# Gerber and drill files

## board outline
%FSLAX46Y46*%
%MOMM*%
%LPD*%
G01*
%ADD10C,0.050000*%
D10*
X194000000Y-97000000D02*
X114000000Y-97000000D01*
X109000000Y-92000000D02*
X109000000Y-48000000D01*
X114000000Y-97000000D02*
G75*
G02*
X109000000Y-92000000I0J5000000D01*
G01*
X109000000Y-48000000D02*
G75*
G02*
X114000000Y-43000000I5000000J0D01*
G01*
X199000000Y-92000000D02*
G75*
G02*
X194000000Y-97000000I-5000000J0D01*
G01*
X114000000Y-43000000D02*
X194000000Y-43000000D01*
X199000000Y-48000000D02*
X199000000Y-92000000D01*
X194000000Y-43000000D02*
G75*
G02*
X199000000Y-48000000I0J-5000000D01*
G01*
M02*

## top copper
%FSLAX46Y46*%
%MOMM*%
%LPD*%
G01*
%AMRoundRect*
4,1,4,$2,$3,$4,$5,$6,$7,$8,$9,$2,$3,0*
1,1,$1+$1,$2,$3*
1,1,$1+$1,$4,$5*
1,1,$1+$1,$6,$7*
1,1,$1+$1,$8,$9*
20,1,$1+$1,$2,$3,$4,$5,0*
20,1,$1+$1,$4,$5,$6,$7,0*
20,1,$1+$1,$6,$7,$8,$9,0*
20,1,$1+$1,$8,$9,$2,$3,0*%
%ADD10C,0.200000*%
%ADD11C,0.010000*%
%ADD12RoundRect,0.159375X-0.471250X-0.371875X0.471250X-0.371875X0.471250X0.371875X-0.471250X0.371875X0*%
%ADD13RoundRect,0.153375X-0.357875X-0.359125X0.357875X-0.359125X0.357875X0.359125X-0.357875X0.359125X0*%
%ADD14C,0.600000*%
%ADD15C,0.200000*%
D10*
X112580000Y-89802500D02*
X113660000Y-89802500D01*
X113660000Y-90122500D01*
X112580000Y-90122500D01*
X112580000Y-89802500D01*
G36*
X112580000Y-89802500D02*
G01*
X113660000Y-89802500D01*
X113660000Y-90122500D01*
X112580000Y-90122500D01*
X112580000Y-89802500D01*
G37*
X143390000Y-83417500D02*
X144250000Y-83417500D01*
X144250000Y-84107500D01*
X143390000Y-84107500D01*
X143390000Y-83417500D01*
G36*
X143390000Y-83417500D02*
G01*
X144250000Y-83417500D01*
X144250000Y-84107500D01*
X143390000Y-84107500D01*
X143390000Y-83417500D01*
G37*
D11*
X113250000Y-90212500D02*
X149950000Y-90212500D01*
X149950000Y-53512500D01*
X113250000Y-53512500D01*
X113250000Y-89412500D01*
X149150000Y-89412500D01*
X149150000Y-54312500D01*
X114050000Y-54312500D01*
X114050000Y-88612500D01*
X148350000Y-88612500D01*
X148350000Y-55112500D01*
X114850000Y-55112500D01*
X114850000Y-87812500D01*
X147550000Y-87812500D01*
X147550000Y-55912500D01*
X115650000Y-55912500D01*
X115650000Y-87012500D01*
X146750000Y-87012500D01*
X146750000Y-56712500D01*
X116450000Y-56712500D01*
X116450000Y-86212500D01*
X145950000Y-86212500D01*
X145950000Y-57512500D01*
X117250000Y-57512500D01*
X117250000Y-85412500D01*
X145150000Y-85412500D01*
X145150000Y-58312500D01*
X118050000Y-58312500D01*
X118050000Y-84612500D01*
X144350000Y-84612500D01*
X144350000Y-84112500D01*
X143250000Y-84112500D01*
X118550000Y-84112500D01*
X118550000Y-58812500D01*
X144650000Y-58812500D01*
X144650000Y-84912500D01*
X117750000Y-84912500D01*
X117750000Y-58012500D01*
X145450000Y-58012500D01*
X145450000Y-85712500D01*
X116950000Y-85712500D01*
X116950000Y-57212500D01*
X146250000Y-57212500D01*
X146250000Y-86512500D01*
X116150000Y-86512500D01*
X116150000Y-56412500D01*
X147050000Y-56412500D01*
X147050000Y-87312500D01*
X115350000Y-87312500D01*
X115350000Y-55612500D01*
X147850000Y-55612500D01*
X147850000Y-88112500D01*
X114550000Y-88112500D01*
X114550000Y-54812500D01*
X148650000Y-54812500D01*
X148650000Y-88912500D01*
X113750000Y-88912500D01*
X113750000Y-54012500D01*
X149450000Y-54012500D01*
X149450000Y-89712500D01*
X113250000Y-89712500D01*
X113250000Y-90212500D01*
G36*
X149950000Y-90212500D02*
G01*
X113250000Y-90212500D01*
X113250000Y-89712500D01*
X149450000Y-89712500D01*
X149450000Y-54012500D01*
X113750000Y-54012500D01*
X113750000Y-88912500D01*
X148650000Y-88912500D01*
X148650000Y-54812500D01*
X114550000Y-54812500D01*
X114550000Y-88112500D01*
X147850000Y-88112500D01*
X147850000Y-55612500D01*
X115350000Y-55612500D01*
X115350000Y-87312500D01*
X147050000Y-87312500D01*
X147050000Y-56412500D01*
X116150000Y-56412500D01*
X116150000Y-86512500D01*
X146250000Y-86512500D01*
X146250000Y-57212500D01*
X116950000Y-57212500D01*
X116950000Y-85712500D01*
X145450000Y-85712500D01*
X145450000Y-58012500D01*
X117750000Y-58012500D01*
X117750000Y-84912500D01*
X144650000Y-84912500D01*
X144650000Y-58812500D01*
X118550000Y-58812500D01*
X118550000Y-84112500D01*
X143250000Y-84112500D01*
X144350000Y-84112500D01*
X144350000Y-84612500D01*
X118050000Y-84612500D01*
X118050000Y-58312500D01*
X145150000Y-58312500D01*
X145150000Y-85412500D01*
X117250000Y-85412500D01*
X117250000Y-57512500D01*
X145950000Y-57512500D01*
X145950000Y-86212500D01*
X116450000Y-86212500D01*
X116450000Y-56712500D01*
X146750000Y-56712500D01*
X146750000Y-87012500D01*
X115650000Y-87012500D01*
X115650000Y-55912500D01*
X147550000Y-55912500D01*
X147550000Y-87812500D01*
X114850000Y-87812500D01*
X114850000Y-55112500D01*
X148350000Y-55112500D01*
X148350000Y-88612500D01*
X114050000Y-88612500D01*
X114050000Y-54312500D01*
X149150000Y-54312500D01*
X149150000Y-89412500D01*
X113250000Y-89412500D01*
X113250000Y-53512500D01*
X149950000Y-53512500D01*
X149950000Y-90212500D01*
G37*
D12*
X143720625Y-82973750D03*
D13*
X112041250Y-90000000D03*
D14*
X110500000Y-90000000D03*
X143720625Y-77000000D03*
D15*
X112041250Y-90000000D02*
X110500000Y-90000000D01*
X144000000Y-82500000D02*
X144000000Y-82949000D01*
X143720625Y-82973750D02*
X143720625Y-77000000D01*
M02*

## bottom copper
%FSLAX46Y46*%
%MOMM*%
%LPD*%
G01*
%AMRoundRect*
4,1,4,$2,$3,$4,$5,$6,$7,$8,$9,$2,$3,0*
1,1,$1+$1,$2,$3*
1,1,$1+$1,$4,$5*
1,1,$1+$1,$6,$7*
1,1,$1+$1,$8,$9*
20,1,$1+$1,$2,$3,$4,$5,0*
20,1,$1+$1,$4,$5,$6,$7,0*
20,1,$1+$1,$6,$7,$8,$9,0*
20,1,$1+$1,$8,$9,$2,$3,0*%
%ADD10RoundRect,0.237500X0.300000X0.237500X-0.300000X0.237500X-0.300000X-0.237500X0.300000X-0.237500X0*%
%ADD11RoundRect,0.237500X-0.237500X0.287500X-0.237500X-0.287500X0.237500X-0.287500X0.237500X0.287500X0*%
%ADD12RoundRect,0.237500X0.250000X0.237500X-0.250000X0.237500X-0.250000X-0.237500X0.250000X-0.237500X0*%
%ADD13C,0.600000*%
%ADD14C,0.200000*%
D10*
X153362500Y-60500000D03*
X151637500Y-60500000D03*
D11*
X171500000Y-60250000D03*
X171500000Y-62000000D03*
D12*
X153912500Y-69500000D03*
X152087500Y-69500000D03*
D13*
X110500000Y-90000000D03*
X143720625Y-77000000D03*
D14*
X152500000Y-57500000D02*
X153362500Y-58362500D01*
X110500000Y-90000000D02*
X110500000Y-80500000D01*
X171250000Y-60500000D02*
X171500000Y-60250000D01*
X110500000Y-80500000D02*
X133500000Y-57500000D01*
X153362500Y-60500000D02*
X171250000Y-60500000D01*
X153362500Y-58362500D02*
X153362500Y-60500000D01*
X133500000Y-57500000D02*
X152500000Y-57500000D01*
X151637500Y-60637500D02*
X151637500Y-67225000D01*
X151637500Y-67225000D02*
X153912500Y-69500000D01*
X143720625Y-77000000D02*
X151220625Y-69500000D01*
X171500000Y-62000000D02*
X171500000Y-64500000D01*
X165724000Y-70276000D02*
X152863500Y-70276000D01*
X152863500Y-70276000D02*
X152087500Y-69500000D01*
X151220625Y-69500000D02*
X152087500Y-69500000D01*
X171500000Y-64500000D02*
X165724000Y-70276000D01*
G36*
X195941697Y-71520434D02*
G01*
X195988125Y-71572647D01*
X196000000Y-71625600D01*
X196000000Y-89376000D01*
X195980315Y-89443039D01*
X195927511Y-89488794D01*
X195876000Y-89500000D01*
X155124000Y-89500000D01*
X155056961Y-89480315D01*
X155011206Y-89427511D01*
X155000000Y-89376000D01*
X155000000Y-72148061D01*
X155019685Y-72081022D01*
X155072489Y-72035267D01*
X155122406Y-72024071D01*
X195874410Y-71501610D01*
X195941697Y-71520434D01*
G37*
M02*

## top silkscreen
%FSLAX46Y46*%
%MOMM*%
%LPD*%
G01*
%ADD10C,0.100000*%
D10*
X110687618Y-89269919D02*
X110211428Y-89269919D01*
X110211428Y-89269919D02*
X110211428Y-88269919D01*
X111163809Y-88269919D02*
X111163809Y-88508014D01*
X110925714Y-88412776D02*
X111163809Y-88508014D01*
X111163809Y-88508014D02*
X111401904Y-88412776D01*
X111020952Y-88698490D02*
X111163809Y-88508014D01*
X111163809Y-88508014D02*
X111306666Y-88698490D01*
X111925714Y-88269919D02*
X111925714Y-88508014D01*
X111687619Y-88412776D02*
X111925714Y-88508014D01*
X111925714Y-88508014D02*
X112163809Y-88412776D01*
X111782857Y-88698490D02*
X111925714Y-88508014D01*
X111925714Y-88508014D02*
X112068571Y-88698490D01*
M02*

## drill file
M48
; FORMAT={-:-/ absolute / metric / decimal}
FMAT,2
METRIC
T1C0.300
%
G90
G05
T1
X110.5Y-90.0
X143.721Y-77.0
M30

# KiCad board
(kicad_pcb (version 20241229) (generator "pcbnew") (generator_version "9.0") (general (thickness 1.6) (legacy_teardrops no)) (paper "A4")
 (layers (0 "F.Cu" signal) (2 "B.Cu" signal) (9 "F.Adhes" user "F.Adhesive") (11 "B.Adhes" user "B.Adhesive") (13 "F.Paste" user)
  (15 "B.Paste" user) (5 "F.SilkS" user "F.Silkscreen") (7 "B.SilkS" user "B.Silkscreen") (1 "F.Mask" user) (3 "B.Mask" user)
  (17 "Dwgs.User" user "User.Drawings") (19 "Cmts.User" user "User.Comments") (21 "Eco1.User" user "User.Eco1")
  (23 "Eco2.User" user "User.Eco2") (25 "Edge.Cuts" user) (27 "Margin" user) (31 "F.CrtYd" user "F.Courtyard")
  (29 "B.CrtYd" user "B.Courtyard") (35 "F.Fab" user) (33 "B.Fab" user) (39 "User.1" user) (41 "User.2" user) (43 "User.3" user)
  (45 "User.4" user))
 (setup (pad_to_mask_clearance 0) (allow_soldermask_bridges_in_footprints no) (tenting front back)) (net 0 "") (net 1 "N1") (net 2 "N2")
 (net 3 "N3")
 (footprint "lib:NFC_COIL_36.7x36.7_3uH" (layer "F.Cu") (at 113.25 90.2125)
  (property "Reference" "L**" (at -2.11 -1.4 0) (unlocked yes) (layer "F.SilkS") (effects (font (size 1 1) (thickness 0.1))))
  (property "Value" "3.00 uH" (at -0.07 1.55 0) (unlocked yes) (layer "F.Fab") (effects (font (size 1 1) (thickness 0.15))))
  (fp_rect (start -0.67 -0.41) (end 0.41 -0.09) (stroke (width 0.2) (type solid)) (fill yes) (layer "F.Cu"))
  (fp_rect (start 30.14 -6.795) (end 31 -6.105) (stroke (width 0.2) (type solid)) (fill yes) (layer "F.Cu"))
  (fp_poly
   (pts (xy 0 0) (xy 36.7 0) (xy 36.7 -36.7) (xy 0 -36.7) (xy 0 -0.8) (xy 35.9 -0.8) (xy 35.9 -35.9) (xy 0.8 -35.9) (xy 0.8 -1.6)
    (xy 35.1 -1.6) (xy 35.1 -35.1) (xy 1.6 -35.1) (xy 1.6 -2.4) (xy 34.3 -2.4) (xy 34.3 -34.3) (xy 2.4 -34.3) (xy 2.4 -3.2) (xy 33.5 -3.2)
    (xy 33.5 -33.5) (xy 3.2 -33.5) (xy 3.2 -4) (xy 32.7 -4) (xy 32.7 -32.7) (xy 4 -32.7) (xy 4 -4.8) (xy 31.9 -4.8) (xy 31.9 -31.9)
    (xy 4.8 -31.9) (xy 4.8 -5.6) (xy 31.1 -5.6) (xy 31.1 -6.1) (xy 30 -6.1) (xy 5.3 -6.1) (xy 5.3 -31.4) (xy 31.4 -31.4) (xy 31.4 -5.3)
    (xy 4.5 -5.3) (xy 4.5 -32.2) (xy 32.2 -32.2) (xy 32.2 -4.5) (xy 3.7 -4.5) (xy 3.7 -33) (xy 33 -33) (xy 33 -3.7) (xy 2.9 -3.7)
    (xy 2.9 -33.8) (xy 33.8 -33.8) (xy 33.8 -2.9) (xy 2.1 -2.9) (xy 2.1 -34.6) (xy 34.6 -34.6) (xy 34.6 -2.1) (xy 1.3 -2.1) (xy 1.3 -35.4)
    (xy 35.4 -35.4) (xy 35.4 -1.3) (xy 0.5 -1.3) (xy 0.5 -36.2) (xy 36.2 -36.2) (xy 36.2 -0.5) (xy 0 -0.5))
   (stroke (width 0.01) (type solid)) (fill yes) (layer "F.Cu"))
  (pad "1" smd roundrect (at 30.470625 -7.23875) (size 1.26125 1.0625) (layers "F.Cu" "F.Mask" "F.Paste") (roundrect_rratio 0.15)
   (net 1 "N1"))
  (pad "2" smd roundrect (at -1.20875 -0.2125) (size 1.0225 1.025) (layers "F.Cu" "F.Mask" "F.Paste") (roundrect_rratio 0.15) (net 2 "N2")))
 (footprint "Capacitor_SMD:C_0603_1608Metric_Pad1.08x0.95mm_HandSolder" (layer "B.Cu") (at 152.5 60.5 180)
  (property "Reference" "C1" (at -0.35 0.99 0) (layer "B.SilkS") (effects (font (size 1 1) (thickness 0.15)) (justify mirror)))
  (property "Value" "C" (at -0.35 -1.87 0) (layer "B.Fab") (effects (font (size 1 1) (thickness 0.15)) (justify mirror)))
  (pad "1" smd roundrect (at -0.8625 0 180) (size 1.075 0.95) (layers "B.Cu" "B.Mask" "B.Paste") (roundrect_rratio 0.25) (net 2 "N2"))
  (pad "2" smd roundrect (at 0.8625 0 180) (size 1.075 0.95) (layers "B.Cu" "B.Mask" "B.Paste") (roundrect_rratio 0.25) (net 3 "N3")))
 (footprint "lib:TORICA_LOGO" (layer "B.Cu") (at 176 54.5 180)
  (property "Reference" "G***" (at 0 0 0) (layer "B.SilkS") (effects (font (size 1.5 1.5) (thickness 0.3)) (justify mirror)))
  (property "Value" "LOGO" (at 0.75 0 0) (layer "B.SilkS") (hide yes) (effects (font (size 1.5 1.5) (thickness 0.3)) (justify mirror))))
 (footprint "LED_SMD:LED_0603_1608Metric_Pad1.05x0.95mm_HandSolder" (layer "B.Cu") (at 171.5 61.125 -90)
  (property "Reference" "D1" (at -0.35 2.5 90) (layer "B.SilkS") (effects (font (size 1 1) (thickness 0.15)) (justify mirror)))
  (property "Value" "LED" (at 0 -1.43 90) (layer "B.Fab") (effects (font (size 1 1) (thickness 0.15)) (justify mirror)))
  (pad "1" smd roundrect (at -0.875 0 270) (size 1.05 0.95) (layers "B.Cu" "B.Mask" "B.Paste") (roundrect_rratio 0.25) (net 2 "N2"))
  (pad "2" smd roundrect (at 0.875 0 270) (size 1.05 0.95) (layers "B.Cu" "B.Mask" "B.Paste") (roundrect_rratio 0.25) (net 1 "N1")))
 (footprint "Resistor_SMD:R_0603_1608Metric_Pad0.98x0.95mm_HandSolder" (layer "B.Cu") (at 153 69.5 180)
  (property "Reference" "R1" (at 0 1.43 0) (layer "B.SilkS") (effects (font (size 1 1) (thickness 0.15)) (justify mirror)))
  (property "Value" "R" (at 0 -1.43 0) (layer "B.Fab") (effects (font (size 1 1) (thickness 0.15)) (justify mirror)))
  (pad "1" smd roundrect (at -0.9125 0 180) (size 0.975 0.95) (layers "B.Cu" "B.Mask" "B.Paste") (roundrect_rratio 0.25) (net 3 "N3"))
  (pad "2" smd roundrect (at 0.9125 0 180) (size 0.975 0.95) (layers "B.Cu" "B.Mask" "B.Paste") (roundrect_rratio 0.25) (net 1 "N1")))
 (gr_line (start 194 97) (end 114 97) (stroke (width 0.05) (type default)) (layer "Edge.Cuts"))
 (gr_line (start 109 92) (end 109 48) (stroke (width 0.05) (type default)) (layer "Edge.Cuts"))
 (gr_arc (start 114 97) (mid 110.464466 95.535534) (end 109 92) (stroke (width 0.05) (type default)) (layer "Edge.Cuts"))
 (gr_arc (start 109 48) (mid 110.464466 44.464466) (end 114 43) (stroke (width 0.05) (type default)) (layer "Edge.Cuts"))
 (gr_arc (start 199 92) (mid 197.535534 95.535534) (end 194 97) (stroke (width 0.05) (type default)) (layer "Edge.Cuts"))
 (gr_line (start 114 43) (end 194 43) (stroke (width 0.05) (type default)) (layer "Edge.Cuts"))
 (gr_line (start 199 48) (end 199 92) (stroke (width 0.05) (type default)) (layer "Edge.Cuts"))
 (gr_arc (start 194 43) (mid 197.535534 44.464466) (end 199 48) (stroke (width 0.05) (type default)) (layer "Edge.Cuts"))
 (segment (start 112.04125 90) (end 110.5 90) (width 0.2) (layer "F.Cu") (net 2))
 (via (at 110.5 90) (size 0.6) (drill 0.3) (layers "F.Cu" "B.Cu") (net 2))
 (segment (start 152.5 57.5) (end 153.3625 58.3625) (width 0.2) (layer "B.Cu") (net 2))
 (segment (start 110.5 90) (end 110.5 80.5) (width 0.2) (layer "B.Cu") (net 2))
 (segment (start 171.25 60.5) (end 171.5 60.25) (width 0.2) (layer "B.Cu") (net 2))
 (segment (start 110.5 80.5) (end 133.5 57.5) (width 0.2) (layer "B.Cu") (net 2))
 (segment (start 153.3625 60.5) (end 171.25 60.5) (width 0.2) (layer "B.Cu") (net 2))
 (segment (start 153.3625 58.3625) (end 153.3625 60.5) (width 0.2) (layer "B.Cu") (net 2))
 (segment (start 133.5 57.5) (end 152.5 57.5) (width 0.2) (layer "B.Cu") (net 2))
 (segment (start 151.6375 60.6375) (end 151.6375 67.225) (width 0.2) (layer "B.Cu") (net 3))
 (segment (start 151.6375 67.225) (end 153.9125 69.5) (width 0.2) (layer "B.Cu") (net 3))
 (segment (start 144 82.5) (end 144 82.949) (width 0.2) (layer "F.Cu") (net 1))
 (segment (start 143.720625 82.97375) (end 143.720625 77) (width 0.2) (layer "F.Cu") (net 1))
 (via (at 143.720625 77) (size 0.6) (drill 0.3) (layers "F.Cu" "B.Cu") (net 1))
 (segment (start 143.720625 77) (end 151.220625 69.5) (width 0.2) (layer "B.Cu") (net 1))
 (segment (start 171.5 62) (end 171.5 64.5) (width 0.2) (layer "B.Cu") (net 1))
 (segment (start 165.724 70.276) (end 152.8635 70.276) (width 0.2) (layer "B.Cu") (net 1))
 (segment (start 152.8635 70.276) (end 152.0875 69.5) (width 0.2) (layer "B.Cu") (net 1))
 (segment (start 151.220625 69.5) (end 152.0875 69.5) (width 0.2) (layer "B.Cu") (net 1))
 (segment (start 171.5 64.5) (end 165.724 70.276) (width 0.2) (layer "B.Cu") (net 1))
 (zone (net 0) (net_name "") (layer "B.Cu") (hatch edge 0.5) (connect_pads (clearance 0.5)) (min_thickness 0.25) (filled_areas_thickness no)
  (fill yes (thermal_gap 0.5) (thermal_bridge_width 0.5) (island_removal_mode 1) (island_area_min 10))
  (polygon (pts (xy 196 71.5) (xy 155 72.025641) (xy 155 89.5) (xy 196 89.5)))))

